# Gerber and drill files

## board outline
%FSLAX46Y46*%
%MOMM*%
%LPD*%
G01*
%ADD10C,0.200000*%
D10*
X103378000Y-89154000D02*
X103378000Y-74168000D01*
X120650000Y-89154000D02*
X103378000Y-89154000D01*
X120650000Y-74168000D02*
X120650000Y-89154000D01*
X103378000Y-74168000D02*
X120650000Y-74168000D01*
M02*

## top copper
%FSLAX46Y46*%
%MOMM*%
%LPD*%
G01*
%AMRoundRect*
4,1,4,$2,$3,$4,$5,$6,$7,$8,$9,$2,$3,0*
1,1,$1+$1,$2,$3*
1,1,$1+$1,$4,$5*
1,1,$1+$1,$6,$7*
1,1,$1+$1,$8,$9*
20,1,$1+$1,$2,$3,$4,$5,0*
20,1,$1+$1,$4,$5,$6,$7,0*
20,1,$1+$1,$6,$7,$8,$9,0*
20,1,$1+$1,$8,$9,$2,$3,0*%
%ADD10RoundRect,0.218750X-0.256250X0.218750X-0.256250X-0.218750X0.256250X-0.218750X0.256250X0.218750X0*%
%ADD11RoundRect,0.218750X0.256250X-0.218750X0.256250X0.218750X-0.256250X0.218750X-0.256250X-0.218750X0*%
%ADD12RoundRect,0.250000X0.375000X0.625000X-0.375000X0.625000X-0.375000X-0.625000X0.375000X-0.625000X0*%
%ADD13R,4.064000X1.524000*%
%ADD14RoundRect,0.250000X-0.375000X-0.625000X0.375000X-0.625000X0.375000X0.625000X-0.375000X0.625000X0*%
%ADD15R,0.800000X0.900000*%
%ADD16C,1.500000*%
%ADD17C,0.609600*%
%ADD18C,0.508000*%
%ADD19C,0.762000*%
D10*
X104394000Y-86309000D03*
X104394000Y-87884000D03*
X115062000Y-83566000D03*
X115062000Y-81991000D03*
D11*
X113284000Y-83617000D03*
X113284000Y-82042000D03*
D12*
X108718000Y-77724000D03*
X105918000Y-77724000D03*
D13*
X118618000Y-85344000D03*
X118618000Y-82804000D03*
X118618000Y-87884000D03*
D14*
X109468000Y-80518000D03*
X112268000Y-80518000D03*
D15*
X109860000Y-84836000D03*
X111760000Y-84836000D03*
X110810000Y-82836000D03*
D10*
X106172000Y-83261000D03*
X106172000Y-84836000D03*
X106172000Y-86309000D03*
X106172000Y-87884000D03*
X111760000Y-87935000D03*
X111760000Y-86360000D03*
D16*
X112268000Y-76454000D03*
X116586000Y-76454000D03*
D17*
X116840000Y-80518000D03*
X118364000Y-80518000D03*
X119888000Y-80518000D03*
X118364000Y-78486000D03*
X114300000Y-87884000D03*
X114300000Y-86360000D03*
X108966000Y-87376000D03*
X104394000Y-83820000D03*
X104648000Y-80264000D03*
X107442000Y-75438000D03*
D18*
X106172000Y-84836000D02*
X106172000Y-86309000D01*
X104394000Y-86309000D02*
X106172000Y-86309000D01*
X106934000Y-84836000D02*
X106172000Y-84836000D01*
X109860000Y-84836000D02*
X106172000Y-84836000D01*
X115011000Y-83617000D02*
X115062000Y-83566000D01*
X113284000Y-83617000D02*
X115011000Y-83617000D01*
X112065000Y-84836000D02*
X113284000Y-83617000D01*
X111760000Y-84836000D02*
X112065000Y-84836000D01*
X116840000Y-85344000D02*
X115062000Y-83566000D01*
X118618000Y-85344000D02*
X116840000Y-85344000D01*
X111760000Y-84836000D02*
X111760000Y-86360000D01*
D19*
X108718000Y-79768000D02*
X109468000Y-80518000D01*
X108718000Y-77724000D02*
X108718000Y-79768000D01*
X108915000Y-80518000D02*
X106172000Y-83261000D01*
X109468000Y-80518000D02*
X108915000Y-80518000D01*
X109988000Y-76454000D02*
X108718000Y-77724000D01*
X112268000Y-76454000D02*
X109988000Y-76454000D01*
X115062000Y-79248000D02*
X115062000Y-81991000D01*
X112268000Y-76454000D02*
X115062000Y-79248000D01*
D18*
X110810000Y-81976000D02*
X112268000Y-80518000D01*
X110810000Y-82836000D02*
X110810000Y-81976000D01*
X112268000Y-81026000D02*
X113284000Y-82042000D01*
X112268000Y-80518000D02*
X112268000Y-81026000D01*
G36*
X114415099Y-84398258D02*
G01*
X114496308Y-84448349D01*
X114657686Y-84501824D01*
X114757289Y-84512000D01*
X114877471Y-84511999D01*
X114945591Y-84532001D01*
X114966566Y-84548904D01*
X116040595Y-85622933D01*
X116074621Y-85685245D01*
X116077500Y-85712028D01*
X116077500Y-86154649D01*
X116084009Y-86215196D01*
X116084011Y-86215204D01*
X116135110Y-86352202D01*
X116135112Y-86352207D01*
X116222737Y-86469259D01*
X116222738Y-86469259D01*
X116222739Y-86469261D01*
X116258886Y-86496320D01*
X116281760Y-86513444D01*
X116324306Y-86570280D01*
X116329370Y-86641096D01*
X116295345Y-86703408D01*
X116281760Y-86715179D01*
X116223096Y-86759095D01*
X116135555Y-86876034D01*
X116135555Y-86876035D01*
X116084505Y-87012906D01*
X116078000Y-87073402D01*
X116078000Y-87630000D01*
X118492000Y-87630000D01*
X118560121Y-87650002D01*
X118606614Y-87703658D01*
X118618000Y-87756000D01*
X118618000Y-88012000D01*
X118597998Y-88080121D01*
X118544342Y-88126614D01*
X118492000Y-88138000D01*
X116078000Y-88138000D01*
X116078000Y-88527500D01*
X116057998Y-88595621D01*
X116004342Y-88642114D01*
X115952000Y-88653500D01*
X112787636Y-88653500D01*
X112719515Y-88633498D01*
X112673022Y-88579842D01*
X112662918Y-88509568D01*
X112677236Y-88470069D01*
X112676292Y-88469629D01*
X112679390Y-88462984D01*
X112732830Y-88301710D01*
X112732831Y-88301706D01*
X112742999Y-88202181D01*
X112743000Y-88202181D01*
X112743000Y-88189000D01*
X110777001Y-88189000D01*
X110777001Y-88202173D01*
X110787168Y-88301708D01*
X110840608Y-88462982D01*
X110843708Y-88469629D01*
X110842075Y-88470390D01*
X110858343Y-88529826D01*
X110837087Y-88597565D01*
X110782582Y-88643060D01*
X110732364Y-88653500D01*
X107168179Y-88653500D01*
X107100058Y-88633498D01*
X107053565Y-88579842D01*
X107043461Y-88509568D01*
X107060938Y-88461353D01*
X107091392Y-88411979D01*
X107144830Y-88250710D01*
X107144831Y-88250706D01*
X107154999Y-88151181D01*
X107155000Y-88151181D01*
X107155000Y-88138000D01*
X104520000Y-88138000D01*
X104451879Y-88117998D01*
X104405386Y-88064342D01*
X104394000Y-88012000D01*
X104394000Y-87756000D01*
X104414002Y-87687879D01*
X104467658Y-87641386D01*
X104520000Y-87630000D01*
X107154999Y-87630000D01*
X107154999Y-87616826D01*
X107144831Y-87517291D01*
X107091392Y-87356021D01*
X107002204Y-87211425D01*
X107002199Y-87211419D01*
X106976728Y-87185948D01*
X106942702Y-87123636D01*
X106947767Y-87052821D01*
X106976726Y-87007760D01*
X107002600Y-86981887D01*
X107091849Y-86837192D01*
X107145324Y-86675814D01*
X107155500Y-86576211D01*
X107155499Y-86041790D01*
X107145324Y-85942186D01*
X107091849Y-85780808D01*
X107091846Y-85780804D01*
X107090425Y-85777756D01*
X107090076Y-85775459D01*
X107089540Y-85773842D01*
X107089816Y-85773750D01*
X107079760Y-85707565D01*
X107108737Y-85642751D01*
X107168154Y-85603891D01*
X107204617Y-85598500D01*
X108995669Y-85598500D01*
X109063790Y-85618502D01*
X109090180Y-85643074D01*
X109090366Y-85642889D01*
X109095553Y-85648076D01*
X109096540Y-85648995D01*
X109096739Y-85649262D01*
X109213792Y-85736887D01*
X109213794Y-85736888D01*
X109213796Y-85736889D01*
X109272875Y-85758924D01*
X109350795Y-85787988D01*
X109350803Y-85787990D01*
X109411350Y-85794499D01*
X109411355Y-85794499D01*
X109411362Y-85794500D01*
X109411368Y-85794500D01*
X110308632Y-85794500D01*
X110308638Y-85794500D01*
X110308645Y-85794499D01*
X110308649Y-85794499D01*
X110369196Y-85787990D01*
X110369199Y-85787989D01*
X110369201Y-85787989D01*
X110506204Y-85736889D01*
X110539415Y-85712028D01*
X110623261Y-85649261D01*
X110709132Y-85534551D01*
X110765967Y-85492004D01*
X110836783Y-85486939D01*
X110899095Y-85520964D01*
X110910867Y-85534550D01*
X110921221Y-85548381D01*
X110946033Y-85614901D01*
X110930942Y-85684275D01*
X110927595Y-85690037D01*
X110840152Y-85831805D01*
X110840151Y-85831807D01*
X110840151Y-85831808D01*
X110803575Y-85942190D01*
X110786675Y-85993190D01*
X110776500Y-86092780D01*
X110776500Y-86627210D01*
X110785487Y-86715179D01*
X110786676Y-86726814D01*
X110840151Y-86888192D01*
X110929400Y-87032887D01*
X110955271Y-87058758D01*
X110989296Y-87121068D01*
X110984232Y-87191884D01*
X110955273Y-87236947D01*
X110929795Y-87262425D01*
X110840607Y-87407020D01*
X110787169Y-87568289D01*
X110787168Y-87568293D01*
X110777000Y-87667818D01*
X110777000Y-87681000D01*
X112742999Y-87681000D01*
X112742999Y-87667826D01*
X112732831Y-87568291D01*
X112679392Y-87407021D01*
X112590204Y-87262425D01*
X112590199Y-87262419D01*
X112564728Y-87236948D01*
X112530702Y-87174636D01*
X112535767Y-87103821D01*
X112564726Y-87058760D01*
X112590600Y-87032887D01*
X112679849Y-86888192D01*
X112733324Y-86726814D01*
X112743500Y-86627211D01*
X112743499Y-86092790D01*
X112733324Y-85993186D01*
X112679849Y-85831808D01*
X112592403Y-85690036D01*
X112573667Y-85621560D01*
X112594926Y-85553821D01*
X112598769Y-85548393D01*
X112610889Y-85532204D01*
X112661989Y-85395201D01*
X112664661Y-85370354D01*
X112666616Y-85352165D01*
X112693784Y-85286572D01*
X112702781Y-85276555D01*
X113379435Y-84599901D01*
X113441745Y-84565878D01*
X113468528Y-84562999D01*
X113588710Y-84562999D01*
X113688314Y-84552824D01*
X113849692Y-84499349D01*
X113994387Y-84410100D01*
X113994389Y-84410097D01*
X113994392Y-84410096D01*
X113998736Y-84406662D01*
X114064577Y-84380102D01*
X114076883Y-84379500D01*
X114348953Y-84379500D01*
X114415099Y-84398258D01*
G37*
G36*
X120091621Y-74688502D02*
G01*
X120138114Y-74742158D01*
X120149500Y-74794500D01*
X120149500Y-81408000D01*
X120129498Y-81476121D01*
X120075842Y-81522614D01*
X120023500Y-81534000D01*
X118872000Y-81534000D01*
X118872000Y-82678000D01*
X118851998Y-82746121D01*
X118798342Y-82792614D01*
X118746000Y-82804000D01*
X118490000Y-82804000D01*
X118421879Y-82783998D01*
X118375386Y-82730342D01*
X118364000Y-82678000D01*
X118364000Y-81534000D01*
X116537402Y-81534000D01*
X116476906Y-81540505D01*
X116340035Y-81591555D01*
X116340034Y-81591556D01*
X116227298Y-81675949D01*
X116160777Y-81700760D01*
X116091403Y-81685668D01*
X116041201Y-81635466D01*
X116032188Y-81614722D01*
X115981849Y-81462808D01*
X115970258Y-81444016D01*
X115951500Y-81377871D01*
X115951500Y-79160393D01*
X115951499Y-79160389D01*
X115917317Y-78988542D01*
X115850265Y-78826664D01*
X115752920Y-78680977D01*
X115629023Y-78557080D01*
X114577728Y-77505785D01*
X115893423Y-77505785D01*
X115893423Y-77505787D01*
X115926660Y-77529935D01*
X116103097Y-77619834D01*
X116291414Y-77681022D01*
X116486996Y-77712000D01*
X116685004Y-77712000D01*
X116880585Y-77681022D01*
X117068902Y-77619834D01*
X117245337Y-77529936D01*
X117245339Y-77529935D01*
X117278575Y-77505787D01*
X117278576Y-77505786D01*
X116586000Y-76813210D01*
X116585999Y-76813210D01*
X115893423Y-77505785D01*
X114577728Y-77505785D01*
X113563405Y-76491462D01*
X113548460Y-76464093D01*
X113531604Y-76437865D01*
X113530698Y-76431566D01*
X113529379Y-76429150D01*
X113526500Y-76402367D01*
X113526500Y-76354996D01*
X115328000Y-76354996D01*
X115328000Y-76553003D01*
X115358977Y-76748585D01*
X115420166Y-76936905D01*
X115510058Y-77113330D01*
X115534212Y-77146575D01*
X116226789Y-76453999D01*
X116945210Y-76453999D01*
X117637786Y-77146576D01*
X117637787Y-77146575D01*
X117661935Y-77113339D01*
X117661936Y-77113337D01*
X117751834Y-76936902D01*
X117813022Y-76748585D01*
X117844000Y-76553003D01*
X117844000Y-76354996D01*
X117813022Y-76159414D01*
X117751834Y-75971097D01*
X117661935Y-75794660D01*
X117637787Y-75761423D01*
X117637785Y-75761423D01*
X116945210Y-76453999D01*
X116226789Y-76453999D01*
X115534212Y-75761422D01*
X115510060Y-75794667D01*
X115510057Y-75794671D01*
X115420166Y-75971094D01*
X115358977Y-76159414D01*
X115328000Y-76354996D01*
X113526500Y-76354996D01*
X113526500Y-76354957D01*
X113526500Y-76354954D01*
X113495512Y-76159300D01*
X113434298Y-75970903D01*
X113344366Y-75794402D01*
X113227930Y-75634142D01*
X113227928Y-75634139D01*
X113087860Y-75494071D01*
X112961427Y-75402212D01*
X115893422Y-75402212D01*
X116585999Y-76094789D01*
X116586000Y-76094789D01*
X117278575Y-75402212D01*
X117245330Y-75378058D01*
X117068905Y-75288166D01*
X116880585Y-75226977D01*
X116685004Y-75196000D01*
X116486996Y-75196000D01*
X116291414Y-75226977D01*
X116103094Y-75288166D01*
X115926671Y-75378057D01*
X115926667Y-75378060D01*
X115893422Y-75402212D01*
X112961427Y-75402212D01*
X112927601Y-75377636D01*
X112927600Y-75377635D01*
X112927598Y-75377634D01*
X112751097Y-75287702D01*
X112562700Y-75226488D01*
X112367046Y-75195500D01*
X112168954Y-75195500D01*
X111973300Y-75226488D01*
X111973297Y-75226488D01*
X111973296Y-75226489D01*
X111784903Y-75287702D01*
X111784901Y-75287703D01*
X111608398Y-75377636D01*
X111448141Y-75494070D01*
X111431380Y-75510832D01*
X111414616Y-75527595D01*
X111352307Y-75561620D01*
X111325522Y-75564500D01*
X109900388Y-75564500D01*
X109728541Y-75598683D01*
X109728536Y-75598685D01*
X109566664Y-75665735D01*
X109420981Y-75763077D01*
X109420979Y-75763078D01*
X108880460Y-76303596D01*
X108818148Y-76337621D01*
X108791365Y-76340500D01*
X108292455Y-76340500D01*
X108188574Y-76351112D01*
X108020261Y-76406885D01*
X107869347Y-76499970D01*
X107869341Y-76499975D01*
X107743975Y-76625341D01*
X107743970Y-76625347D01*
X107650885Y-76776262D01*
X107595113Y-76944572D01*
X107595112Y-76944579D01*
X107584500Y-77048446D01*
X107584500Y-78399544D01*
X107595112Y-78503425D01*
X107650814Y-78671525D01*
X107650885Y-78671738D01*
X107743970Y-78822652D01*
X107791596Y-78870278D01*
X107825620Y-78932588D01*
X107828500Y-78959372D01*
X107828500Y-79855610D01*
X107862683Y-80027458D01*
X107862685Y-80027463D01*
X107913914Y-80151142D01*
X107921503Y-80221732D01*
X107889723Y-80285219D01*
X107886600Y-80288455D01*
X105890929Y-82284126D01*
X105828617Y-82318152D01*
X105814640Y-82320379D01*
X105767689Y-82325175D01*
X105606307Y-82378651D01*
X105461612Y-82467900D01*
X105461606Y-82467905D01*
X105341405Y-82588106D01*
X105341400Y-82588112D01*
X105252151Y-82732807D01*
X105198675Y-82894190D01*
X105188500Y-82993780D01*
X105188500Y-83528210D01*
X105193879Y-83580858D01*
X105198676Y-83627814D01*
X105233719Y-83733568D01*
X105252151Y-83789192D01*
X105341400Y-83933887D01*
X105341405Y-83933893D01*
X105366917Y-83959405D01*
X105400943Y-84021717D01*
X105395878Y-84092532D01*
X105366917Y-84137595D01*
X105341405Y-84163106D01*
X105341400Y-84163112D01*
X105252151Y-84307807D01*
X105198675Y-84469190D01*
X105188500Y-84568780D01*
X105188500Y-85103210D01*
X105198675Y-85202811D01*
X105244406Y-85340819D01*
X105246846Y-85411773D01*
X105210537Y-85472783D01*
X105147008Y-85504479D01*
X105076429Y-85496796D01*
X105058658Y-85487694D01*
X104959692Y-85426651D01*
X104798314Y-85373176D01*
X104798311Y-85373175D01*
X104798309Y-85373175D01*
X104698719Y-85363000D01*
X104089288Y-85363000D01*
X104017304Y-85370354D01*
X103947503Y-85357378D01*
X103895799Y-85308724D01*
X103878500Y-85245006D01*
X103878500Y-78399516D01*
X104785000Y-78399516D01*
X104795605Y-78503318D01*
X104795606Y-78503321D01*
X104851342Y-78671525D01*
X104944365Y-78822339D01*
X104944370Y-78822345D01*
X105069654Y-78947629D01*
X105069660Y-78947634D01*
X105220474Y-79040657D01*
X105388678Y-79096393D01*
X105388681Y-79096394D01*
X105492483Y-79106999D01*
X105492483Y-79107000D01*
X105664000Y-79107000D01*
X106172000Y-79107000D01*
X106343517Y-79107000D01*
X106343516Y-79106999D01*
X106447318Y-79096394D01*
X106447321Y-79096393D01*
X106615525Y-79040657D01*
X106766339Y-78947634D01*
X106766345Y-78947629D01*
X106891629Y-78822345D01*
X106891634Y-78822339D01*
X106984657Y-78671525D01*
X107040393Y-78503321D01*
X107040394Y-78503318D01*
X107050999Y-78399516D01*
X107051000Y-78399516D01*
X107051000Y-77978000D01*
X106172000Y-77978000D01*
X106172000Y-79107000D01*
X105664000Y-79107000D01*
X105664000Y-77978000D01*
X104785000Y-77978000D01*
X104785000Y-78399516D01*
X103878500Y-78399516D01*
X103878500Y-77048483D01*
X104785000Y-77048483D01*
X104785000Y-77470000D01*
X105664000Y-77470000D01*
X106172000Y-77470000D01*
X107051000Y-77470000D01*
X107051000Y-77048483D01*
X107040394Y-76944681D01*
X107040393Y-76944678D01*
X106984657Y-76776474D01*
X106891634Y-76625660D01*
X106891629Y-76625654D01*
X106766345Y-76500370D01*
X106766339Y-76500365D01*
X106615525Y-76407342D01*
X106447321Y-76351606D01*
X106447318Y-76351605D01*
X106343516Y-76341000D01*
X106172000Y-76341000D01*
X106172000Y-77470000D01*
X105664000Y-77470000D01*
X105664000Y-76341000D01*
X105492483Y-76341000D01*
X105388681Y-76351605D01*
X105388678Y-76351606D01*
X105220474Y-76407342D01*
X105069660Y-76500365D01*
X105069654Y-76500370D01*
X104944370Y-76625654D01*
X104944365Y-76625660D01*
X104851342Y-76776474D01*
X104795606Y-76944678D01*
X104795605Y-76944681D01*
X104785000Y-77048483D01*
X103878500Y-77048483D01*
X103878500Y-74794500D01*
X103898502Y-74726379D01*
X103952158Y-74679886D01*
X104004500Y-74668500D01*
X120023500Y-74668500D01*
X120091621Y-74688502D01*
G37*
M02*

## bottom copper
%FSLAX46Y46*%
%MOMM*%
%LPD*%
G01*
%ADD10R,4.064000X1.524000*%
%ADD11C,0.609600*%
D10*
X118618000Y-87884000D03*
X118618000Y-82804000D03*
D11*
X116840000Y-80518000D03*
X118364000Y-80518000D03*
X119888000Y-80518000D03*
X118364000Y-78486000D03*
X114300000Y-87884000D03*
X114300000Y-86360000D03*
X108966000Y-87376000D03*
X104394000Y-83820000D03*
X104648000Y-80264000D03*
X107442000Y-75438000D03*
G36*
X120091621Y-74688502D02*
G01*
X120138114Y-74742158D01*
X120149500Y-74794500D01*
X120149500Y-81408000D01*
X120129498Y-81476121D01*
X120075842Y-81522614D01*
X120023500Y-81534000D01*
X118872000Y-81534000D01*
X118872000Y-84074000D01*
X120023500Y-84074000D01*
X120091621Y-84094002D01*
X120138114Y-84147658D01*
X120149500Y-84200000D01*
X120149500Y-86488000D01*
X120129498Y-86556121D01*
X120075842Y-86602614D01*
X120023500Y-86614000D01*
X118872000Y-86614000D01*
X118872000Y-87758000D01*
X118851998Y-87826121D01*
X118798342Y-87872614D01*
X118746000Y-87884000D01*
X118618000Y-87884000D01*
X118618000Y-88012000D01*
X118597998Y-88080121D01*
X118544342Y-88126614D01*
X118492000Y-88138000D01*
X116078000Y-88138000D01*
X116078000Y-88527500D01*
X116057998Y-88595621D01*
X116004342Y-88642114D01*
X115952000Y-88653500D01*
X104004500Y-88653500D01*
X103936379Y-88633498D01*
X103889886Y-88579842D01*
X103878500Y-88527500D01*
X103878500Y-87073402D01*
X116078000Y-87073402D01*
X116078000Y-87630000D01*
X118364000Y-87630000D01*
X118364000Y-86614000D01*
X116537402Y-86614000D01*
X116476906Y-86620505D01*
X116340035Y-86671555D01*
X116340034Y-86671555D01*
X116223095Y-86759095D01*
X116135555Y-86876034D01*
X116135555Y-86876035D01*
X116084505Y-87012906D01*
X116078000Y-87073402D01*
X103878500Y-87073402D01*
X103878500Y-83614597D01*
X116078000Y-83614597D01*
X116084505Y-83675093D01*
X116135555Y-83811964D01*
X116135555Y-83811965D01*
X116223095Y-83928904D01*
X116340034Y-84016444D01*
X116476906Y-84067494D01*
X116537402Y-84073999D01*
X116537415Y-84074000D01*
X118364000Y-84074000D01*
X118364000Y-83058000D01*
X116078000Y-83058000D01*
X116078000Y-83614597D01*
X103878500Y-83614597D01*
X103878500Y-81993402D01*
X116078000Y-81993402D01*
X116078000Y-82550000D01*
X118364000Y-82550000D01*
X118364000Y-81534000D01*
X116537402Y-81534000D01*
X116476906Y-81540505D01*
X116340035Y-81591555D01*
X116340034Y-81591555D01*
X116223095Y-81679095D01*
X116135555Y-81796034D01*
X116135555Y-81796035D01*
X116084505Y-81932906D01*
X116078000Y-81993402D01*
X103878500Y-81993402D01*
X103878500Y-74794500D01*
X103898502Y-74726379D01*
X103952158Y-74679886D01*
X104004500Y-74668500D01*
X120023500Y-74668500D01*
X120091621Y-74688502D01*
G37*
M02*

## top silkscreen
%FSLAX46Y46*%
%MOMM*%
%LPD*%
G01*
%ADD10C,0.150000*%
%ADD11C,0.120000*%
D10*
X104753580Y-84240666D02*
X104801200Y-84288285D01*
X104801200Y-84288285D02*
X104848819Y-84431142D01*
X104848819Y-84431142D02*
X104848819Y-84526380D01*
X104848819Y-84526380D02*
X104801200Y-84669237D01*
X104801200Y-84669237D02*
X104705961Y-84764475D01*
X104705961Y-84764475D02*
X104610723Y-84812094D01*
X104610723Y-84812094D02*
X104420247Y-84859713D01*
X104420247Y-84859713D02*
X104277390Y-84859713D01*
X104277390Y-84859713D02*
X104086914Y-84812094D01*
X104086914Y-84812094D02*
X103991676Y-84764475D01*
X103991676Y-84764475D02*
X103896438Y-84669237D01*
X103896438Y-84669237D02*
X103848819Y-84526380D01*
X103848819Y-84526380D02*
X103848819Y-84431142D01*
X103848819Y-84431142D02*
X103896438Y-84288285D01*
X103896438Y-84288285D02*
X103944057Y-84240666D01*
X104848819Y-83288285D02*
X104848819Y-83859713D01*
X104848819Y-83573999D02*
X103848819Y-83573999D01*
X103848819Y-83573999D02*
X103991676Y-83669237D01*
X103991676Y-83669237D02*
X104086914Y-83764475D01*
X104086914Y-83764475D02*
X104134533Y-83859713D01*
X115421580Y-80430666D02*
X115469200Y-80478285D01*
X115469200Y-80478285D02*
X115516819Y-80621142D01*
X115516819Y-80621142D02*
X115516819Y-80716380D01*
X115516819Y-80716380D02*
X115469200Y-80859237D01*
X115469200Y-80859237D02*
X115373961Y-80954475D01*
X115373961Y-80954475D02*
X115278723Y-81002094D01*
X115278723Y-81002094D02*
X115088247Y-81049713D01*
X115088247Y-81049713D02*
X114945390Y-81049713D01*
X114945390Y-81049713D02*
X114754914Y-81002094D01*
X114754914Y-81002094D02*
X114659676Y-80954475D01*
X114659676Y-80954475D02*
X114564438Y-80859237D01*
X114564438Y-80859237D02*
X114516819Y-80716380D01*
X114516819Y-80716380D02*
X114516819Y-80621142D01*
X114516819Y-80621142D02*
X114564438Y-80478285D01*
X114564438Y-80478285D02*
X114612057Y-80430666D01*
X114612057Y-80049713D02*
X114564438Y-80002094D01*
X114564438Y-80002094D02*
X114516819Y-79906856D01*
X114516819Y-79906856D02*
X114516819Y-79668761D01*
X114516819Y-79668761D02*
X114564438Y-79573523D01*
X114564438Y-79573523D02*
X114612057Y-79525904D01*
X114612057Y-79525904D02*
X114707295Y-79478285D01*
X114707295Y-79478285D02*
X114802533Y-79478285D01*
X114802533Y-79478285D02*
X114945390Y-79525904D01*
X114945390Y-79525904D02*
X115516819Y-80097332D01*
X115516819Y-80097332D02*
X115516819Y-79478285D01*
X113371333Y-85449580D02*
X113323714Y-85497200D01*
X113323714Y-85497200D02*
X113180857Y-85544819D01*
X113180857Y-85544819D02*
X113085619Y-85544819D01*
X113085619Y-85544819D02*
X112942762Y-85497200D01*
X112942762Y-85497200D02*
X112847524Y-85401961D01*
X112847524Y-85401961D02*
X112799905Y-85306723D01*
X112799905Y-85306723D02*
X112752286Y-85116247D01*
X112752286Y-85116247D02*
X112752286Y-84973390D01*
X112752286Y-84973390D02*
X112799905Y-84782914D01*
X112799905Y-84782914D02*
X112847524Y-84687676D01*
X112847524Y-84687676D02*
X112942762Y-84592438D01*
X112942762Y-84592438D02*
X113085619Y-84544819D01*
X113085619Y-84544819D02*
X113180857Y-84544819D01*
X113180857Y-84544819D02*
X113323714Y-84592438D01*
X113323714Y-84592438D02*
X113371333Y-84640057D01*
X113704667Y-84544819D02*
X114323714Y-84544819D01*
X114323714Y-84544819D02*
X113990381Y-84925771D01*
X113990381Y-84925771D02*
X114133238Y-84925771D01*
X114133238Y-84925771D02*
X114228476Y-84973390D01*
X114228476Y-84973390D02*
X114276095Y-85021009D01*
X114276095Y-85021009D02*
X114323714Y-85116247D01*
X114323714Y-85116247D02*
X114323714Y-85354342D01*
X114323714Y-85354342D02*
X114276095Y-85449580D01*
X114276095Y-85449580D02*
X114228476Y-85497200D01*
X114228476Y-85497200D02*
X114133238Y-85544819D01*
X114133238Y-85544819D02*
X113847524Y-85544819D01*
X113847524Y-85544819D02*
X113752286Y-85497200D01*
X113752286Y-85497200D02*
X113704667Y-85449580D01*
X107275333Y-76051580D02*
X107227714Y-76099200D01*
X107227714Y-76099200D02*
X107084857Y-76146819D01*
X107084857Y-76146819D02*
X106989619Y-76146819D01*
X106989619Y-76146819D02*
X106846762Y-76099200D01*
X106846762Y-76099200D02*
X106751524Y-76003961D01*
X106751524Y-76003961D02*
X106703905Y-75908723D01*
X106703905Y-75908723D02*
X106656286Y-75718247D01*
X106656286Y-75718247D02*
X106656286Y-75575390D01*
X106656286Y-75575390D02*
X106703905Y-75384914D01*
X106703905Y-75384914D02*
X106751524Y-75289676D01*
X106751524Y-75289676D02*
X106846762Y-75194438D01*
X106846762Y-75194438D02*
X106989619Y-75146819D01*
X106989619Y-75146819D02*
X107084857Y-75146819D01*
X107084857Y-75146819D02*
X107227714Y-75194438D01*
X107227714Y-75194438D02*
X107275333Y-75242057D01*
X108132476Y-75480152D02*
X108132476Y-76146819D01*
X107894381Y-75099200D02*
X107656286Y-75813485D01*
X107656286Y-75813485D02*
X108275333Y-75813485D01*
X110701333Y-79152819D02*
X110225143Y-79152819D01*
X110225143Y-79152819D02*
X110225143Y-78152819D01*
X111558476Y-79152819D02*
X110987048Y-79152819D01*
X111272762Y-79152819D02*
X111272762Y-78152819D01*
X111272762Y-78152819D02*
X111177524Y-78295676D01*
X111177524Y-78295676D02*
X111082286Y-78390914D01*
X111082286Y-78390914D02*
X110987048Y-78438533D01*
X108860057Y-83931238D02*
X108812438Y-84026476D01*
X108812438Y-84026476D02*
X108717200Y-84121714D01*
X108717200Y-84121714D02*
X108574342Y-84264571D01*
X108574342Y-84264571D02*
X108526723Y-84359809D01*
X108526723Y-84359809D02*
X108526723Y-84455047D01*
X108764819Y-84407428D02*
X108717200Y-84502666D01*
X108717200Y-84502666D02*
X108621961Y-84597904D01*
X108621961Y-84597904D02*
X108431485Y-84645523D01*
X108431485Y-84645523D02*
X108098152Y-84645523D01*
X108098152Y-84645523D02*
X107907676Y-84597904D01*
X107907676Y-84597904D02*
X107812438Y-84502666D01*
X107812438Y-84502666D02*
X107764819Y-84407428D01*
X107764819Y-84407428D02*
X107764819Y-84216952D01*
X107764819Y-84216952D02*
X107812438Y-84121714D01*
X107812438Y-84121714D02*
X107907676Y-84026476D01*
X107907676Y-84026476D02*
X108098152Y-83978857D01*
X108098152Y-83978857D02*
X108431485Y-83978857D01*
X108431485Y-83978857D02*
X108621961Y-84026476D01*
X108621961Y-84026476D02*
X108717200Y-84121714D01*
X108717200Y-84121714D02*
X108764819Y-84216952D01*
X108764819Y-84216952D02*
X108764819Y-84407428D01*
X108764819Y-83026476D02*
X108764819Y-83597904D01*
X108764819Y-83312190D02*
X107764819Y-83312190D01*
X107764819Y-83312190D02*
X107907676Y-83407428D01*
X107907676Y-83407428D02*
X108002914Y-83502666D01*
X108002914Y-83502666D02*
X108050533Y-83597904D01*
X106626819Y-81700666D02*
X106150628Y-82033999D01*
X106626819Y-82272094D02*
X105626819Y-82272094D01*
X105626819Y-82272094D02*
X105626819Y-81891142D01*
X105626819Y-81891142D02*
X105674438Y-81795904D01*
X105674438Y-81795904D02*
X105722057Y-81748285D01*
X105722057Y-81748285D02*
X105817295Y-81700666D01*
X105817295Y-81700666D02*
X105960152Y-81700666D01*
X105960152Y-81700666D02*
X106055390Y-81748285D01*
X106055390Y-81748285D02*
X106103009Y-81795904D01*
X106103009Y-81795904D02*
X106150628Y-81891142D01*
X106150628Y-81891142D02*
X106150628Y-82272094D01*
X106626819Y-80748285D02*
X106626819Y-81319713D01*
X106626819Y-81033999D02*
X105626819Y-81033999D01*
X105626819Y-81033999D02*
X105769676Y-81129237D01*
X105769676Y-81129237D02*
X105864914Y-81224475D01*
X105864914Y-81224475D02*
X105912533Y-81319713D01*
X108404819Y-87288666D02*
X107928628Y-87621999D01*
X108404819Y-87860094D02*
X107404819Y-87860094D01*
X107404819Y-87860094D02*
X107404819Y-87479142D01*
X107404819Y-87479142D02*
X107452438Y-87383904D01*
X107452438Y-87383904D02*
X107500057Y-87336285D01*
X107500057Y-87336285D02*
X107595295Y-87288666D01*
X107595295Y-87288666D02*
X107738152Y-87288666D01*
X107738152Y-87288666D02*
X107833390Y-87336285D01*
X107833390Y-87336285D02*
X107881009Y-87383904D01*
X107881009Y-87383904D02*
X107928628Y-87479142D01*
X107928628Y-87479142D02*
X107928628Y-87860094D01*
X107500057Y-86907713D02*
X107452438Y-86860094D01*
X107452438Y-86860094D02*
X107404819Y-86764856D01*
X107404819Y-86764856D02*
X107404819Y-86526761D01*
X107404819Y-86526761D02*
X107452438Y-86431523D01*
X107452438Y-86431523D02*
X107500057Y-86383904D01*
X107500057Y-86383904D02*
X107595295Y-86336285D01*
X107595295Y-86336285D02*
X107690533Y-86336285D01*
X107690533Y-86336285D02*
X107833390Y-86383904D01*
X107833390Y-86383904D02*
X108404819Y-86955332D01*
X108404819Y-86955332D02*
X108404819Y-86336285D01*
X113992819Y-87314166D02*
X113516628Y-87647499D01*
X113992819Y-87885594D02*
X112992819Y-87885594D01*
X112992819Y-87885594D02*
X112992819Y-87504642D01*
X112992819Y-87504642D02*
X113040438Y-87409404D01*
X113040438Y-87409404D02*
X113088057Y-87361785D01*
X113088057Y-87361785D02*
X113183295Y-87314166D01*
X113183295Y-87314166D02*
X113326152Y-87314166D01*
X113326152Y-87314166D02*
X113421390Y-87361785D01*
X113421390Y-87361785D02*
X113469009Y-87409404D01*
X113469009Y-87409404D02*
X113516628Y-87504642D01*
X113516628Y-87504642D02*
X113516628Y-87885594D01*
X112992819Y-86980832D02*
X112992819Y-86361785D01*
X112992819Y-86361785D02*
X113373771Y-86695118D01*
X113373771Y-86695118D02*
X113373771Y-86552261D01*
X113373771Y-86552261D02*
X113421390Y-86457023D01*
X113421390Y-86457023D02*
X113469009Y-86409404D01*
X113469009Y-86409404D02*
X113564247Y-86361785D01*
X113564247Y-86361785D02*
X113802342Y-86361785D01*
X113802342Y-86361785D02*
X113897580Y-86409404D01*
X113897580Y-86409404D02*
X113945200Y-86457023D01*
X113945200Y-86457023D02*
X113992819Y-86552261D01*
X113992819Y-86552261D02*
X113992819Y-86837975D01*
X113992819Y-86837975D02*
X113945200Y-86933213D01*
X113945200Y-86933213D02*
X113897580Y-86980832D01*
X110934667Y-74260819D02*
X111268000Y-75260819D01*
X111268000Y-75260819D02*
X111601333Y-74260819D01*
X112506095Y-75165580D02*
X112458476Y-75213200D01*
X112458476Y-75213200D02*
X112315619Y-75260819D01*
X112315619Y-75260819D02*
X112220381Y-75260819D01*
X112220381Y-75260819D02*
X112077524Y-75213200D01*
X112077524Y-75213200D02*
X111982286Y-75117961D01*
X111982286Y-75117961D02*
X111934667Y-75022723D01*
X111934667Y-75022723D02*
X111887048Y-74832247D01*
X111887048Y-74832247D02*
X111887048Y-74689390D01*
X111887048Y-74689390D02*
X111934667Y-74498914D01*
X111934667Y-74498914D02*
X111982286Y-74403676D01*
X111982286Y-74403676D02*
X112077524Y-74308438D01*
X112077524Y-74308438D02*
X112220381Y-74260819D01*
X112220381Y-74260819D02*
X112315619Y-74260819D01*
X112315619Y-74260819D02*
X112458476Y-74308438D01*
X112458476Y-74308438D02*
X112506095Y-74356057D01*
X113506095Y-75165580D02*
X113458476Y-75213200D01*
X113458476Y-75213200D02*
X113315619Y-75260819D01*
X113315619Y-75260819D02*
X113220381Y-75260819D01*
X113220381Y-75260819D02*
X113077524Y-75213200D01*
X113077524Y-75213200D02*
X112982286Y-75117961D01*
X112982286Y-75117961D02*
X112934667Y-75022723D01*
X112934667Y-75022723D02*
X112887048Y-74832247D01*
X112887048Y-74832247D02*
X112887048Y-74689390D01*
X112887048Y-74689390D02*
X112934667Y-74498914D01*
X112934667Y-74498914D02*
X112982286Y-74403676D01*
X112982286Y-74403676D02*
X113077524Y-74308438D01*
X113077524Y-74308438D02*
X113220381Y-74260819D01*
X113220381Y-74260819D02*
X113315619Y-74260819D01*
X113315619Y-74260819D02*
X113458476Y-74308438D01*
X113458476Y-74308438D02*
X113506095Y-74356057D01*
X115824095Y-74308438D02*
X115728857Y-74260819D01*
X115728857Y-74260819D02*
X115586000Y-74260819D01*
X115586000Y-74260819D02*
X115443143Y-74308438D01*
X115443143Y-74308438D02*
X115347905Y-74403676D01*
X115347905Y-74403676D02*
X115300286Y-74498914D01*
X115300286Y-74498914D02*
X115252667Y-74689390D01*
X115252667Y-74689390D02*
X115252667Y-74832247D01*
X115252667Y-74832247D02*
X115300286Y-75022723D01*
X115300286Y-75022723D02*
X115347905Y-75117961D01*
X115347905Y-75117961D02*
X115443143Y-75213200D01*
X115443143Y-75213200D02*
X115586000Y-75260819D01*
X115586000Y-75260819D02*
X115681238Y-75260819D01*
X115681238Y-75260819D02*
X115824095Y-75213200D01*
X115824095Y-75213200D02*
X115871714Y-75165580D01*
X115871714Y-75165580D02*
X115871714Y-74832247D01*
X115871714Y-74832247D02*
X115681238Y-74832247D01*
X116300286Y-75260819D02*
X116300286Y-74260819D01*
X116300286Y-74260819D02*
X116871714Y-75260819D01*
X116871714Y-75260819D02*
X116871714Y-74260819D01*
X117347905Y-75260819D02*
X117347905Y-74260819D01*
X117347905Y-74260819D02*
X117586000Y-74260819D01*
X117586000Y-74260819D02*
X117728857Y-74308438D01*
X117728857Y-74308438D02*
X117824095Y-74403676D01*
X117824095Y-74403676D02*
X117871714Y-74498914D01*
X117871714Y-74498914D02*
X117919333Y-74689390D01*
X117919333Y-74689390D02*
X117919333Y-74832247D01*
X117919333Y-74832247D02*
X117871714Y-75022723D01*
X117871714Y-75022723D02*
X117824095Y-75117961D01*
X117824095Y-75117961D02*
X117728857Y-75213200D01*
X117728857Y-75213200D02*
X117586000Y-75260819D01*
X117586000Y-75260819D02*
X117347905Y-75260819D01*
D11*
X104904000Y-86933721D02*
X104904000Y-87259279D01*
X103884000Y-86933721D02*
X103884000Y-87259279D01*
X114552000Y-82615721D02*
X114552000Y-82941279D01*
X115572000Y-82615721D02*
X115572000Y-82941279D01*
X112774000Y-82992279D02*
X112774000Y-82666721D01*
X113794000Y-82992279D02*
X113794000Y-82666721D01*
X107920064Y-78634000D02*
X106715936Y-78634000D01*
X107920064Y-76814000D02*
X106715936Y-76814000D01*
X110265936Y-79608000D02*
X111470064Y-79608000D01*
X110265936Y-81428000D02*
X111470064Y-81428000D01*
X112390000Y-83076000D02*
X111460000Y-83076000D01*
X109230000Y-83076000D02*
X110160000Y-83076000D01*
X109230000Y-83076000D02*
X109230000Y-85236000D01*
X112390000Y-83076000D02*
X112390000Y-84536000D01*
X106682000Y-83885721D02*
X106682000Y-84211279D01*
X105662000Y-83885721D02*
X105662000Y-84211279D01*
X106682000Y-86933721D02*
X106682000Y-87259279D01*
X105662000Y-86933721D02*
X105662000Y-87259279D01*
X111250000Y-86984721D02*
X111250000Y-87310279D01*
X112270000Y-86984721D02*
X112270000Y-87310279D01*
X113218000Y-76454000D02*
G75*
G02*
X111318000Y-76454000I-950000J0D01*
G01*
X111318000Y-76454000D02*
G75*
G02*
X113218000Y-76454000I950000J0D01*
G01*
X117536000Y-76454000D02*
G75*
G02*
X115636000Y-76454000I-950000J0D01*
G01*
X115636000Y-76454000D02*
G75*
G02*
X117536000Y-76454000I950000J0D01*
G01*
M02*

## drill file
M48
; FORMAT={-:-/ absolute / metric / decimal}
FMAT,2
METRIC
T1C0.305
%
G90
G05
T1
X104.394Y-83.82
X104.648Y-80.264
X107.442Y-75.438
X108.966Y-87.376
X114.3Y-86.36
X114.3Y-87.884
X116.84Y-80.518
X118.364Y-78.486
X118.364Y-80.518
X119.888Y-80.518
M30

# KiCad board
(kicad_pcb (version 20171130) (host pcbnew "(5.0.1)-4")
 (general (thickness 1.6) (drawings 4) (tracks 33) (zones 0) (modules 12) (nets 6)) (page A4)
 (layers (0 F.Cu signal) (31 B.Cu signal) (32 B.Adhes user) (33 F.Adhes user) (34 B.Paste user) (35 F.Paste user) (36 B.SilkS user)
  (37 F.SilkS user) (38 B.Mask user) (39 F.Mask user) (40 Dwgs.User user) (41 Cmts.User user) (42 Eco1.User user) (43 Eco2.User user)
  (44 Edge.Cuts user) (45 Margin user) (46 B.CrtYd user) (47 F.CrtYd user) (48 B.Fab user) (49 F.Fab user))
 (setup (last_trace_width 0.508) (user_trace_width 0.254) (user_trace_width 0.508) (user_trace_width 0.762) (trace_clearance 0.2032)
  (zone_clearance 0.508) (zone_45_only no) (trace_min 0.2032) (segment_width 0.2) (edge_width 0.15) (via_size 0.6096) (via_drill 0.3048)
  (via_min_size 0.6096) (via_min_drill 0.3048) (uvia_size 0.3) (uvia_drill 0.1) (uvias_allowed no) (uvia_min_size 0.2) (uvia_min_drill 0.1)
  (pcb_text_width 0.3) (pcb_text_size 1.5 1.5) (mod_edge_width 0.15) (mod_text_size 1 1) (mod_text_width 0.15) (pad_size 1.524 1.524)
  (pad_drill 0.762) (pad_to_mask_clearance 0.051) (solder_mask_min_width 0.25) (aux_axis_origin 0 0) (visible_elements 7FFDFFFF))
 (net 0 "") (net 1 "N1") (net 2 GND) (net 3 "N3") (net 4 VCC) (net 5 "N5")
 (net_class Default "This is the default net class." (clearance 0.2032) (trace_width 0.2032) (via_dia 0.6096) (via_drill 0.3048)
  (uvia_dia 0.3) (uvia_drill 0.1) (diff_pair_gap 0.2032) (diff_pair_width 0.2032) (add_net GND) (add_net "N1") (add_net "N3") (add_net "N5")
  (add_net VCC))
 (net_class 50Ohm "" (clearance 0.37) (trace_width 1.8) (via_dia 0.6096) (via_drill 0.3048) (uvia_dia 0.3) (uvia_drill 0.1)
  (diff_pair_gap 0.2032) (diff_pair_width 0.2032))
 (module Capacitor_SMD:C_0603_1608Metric (layer F.Cu) (at 104.394 87.0965 270)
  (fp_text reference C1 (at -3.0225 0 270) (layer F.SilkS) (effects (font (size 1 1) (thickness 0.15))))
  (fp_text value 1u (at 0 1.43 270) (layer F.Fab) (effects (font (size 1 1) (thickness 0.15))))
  (fp_line (start -0.162779 -0.51) (end 0.162779 -0.51) (layer F.SilkS) (width 0.12))
  (fp_line (start -0.162779 0.51) (end 0.162779 0.51) (layer F.SilkS) (width 0.12))
  (pad 1 smd roundrect (at -0.7875 0 270) (size 0.875 0.95) (layers F.Cu F.Paste F.Mask) (roundrect_rratio 0.25) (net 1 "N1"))
  (pad 2 smd roundrect (at 0.7875 0 270) (size 0.875 0.95) (layers F.Cu F.Paste F.Mask) (roundrect_rratio 0.25) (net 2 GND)))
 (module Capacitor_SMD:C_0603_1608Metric (layer F.Cu) (at 115.062 82.7785 270)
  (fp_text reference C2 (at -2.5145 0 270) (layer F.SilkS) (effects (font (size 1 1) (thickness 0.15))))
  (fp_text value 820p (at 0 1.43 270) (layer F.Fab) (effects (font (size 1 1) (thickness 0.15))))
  (fp_line (start -0.162779 0.51) (end 0.162779 0.51) (layer F.SilkS) (width 0.12))
  (fp_line (start -0.162779 -0.51) (end 0.162779 -0.51) (layer F.SilkS) (width 0.12))
  (pad 2 smd roundrect (at 0.7875 0 270) (size 0.875 0.95) (layers F.Cu F.Paste F.Mask) (roundrect_rratio 0.25) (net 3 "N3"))
  (pad 1 smd roundrect (at -0.7875 0 270) (size 0.875 0.95) (layers F.Cu F.Paste F.Mask) (roundrect_rratio 0.25) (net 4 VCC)))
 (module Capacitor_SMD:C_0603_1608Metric (layer F.Cu) (at 113.284 82.8295 90)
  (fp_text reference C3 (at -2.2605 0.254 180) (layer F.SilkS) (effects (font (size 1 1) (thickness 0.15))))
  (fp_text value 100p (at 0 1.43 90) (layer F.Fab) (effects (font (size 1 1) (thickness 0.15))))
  (fp_line (start -0.162779 -0.51) (end 0.162779 -0.51) (layer F.SilkS) (width 0.12))
  (fp_line (start -0.162779 0.51) (end 0.162779 0.51) (layer F.SilkS) (width 0.12))
  (pad 1 smd roundrect (at -0.7875 0 90) (size 0.875 0.95) (layers F.Cu F.Paste F.Mask) (roundrect_rratio 0.25) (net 3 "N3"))
  (pad 2 smd roundrect (at 0.7875 0 90) (size 0.875 0.95) (layers F.Cu F.Paste F.Mask) (roundrect_rratio 0.25) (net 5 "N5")))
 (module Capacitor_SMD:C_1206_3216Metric (layer F.Cu) (at 107.318 77.724 180)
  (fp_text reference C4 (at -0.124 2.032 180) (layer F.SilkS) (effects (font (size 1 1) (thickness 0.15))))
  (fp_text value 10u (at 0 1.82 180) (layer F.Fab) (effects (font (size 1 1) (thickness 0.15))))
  (fp_line (start -0.602064 -0.91) (end 0.602064 -0.91) (layer F.SilkS) (width 0.12))
  (fp_line (start -0.602064 0.91) (end 0.602064 0.91) (layer F.SilkS) (width 0.12))
  (pad 1 smd roundrect (at -1.4 0 180) (size 1.25 1.75) (layers F.Cu F.Paste F.Mask) (roundrect_rratio 0.2) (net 4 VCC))
  (pad 2 smd roundrect (at 1.4 0 180) (size 1.25 1.75) (layers F.Cu F.Paste F.Mask) (roundrect_rratio 0.2) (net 2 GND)))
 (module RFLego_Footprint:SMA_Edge (layer F.Cu) (at 116.586 85.344)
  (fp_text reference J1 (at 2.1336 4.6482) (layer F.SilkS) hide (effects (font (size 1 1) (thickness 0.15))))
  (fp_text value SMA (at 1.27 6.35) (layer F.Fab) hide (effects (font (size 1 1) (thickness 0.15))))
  (pad 1 smd rect (at 2.032 0) (size 4.064 1.524) (layers F.Cu F.Mask) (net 3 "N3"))
  (pad 2 smd rect (at 2.032 -2.54) (size 4.064 1.524) (layers F.Cu F.Mask) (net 2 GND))
  (pad 2 smd rect (at 2.032 2.54) (size 4.064 1.524) (layers B.Cu B.Mask) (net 2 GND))
  (pad 2 smd rect (at 2.032 -2.54) (size 4.064 1.524) (layers B.Cu B.Mask) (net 2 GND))
  (pad 2 smd rect (at 2.032 2.54) (size 4.064 1.524) (layers F.Cu F.Mask) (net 2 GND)))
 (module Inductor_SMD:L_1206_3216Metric (layer F.Cu) (at 110.868 80.518)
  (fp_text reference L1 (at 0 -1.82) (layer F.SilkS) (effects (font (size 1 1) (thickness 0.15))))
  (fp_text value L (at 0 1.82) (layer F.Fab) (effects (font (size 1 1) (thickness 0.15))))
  (fp_line (start -0.602064 -0.91) (end 0.602064 -0.91) (layer F.SilkS) (width 0.12))
  (fp_line (start -0.602064 0.91) (end 0.602064 0.91) (layer F.SilkS) (width 0.12))
  (pad 1 smd roundrect (at -1.4 0) (size 1.25 1.75) (layers F.Cu F.Paste F.Mask) (roundrect_rratio 0.2) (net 4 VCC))
  (pad 2 smd roundrect (at 1.4 0) (size 1.25 1.75) (layers F.Cu F.Paste F.Mask) (roundrect_rratio 0.2) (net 5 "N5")))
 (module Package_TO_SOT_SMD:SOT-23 (layer F.Cu) (at 110.81 83.836 90)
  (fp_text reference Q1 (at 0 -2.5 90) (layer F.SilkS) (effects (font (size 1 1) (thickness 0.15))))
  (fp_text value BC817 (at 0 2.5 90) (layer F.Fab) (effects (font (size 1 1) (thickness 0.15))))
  (fp_line (start 0.76 1.58) (end 0.76 0.65) (layer F.SilkS) (width 0.12))
  (fp_line (start 0.76 -1.58) (end 0.76 -0.65) (layer F.SilkS) (width 0.12))
  (fp_line (start 0.76 -1.58) (end -1.4 -1.58) (layer F.SilkS) (width 0.12))
  (fp_line (start 0.76 1.58) (end -0.7 1.58) (layer F.SilkS) (width 0.12))
  (pad 1 smd rect (at -1 -0.95 90) (size 0.9 0.8) (layers F.Cu F.Paste F.Mask) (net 1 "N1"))
  (pad 2 smd rect (at -1 0.95 90) (size 0.9 0.8) (layers F.Cu F.Paste F.Mask) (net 3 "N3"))
  (pad 3 smd rect (at 1 0 90) (size 0.9 0.8) (layers F.Cu F.Paste F.Mask) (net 5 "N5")))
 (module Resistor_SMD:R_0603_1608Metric (layer F.Cu) (at 106.172 84.0485 270)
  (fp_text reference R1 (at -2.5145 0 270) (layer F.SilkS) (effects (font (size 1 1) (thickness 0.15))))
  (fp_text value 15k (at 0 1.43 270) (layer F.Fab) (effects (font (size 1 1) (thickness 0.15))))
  (fp_line (start -0.162779 -0.51) (end 0.162779 -0.51) (layer F.SilkS) (width 0.12))
  (fp_line (start -0.162779 0.51) (end 0.162779 0.51) (layer F.SilkS) (width 0.12))
  (pad 1 smd roundrect (at -0.7875 0 270) (size 0.875 0.95) (layers F.Cu F.Paste F.Mask) (roundrect_rratio 0.25) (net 4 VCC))
  (pad 2 smd roundrect (at 0.7875 0 270) (size 0.875 0.95) (layers F.Cu F.Paste F.Mask) (roundrect_rratio 0.25) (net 1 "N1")))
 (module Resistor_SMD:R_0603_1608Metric (layer F.Cu) (at 106.172 87.0965 270)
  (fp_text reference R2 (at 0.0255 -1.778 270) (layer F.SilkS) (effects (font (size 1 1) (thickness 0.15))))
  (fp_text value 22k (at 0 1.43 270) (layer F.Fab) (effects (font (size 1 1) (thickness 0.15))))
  (fp_line (start -0.162779 -0.51) (end 0.162779 -0.51) (layer F.SilkS) (width 0.12))
  (fp_line (start -0.162779 0.51) (end 0.162779 0.51) (layer F.SilkS) (width 0.12))
  (pad 1 smd roundrect (at -0.7875 0 270) (size 0.875 0.95) (layers F.Cu F.Paste F.Mask) (roundrect_rratio 0.25) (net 1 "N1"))
  (pad 2 smd roundrect (at 0.7875 0 270) (size 0.875 0.95) (layers F.Cu F.Paste F.Mask) (roundrect_rratio 0.25) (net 2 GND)))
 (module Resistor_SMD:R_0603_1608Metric (layer F.Cu) (at 111.76 87.1475 270)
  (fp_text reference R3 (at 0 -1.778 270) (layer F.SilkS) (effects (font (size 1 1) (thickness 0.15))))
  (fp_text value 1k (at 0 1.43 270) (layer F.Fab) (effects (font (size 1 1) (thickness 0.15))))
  (fp_line (start -0.162779 0.51) (end 0.162779 0.51) (layer F.SilkS) (width 0.12))
  (fp_line (start -0.162779 -0.51) (end 0.162779 -0.51) (layer F.SilkS) (width 0.12))
  (pad 2 smd roundrect (at 0.7875 0 270) (size 0.875 0.95) (layers F.Cu F.Paste F.Mask) (roundrect_rratio 0.25) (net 2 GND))
  (pad 1 smd roundrect (at -0.7875 0 270) (size 0.875 0.95) (layers F.Cu F.Paste F.Mask) (roundrect_rratio 0.25) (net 3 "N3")))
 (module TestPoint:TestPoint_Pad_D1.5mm (layer F.Cu) (at 112.268 76.454)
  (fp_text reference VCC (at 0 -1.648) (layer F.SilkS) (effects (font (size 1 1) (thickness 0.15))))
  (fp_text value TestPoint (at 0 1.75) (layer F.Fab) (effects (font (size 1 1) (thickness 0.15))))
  (fp_circle (center 0 0) (end 0 0.95) (layer F.SilkS) (width 0.12))
  (pad 1 smd circle (at 0 0) (size 1.5 1.5) (layers F.Cu F.Mask) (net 4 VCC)))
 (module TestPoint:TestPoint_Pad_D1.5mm (layer F.Cu) (at 116.586 76.454)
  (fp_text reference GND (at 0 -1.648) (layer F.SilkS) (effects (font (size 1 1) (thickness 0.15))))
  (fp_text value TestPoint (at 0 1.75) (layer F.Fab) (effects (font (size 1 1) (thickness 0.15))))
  (fp_circle (center 0 0) (end 0 0.95) (layer F.SilkS) (width 0.12))
  (pad 1 smd circle (at 0 0) (size 1.5 1.5) (layers F.Cu F.Mask) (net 2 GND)))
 (gr_line (start 103.378 89.154) (end 103.378 74.168) (layer Edge.Cuts) (width 0.2))
 (gr_line (start 120.65 89.154) (end 103.378 89.154) (layer Edge.Cuts) (width 0.2))
 (gr_line (start 120.65 74.168) (end 120.65 89.154) (layer Edge.Cuts) (width 0.2))
 (gr_line (start 103.378 74.168) (end 120.65 74.168) (layer Edge.Cuts) (width 0.2))
 (segment (start 106.172 84.836) (end 106.172 86.309) (width 0.508) (layer F.Cu) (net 1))
 (segment (start 104.394 86.309) (end 106.172 86.309) (width 0.508) (layer F.Cu) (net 1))
 (segment (start 106.934 84.836) (end 106.172 84.836) (width 0.508) (layer F.Cu) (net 1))
 (segment (start 109.86 84.836) (end 106.172 84.836) (width 0.508) (layer F.Cu) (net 1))
 (via (at 116.84 80.518) (size 0.6096) (drill 0.3048) (layers F.Cu B.Cu) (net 2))
 (via (at 118.364 80.518) (size 0.6096) (drill 0.3048) (layers F.Cu B.Cu) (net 2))
 (via (at 119.888 80.518) (size 0.6096) (drill 0.3048) (layers F.Cu B.Cu) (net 2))
 (via (at 118.364 78.486) (size 0.6096) (drill 0.3048) (layers F.Cu B.Cu) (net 2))
 (via (at 114.3 87.884) (size 0.6096) (drill 0.3048) (layers F.Cu B.Cu) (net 2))
 (via (at 114.3 86.36) (size 0.6096) (drill 0.3048) (layers F.Cu B.Cu) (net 2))
 (via (at 108.966 87.376) (size 0.6096) (drill 0.3048) (layers F.Cu B.Cu) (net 2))
 (via (at 104.394 83.82) (size 0.6096) (drill 0.3048) (layers F.Cu B.Cu) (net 2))
 (via (at 104.648 80.264) (size 0.6096) (drill 0.3048) (layers F.Cu B.Cu) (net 2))
 (via (at 107.442 75.438) (size 0.6096) (drill 0.3048) (layers F.Cu B.Cu) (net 2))
 (segment (start 115.011 83.617) (end 115.062 83.566) (width 0.508) (layer F.Cu) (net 3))
 (segment (start 113.284 83.617) (end 115.011 83.617) (width 0.508) (layer F.Cu) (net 3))
 (segment (start 112.065 84.836) (end 113.284 83.617) (width 0.508) (layer F.Cu) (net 3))
 (segment (start 111.76 84.836) (end 112.065 84.836) (width 0.508) (layer F.Cu) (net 3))
 (segment (start 116.84 85.344) (end 115.062 83.566) (width 0.508) (layer F.Cu) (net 3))
 (segment (start 118.618 85.344) (end 116.84 85.344) (width 0.508) (layer F.Cu) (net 3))
 (segment (start 111.76 84.836) (end 111.76 86.36) (width 0.508) (layer F.Cu) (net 3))
 (segment (start 108.718 79.768) (end 109.468 80.518) (width 0.762) (layer F.Cu) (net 4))
 (segment (start 108.718 77.724) (end 108.718 79.768) (width 0.762) (layer F.Cu) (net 4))
 (segment (start 108.915 80.518) (end 106.172 83.261) (width 0.762) (layer F.Cu) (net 4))
 (segment (start 109.468 80.518) (end 108.915 80.518) (width 0.762) (layer F.Cu) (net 4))
 (segment (start 109.988 76.454) (end 108.718 77.724) (width 0.762) (layer F.Cu) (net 4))
 (segment (start 112.268 76.454) (end 109.988 76.454) (width 0.762) (layer F.Cu) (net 4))
 (segment (start 115.062 79.248) (end 115.062 81.991) (width 0.762) (layer F.Cu) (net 4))
 (segment (start 112.268 76.454) (end 115.062 79.248) (width 0.762) (layer F.Cu) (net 4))
 (segment (start 110.81 81.976) (end 112.268 80.518) (width 0.508) (layer F.Cu) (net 5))
 (segment (start 110.81 82.836) (end 110.81 81.976) (width 0.508) (layer F.Cu) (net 5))
 (segment (start 112.268 81.026) (end 113.284 82.042) (width 0.508) (layer F.Cu) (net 5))
 (segment (start 112.268 80.518) (end 112.268 81.026) (width 0.508) (layer F.Cu) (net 5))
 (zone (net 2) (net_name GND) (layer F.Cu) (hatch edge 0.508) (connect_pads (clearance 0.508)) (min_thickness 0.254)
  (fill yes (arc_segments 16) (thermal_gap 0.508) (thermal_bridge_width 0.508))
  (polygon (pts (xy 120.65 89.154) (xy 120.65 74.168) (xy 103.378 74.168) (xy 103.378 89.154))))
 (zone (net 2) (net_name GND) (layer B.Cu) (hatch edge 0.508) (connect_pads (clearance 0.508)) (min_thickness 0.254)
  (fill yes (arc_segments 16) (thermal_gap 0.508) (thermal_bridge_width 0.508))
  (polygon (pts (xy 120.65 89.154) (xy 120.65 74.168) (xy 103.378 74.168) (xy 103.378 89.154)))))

